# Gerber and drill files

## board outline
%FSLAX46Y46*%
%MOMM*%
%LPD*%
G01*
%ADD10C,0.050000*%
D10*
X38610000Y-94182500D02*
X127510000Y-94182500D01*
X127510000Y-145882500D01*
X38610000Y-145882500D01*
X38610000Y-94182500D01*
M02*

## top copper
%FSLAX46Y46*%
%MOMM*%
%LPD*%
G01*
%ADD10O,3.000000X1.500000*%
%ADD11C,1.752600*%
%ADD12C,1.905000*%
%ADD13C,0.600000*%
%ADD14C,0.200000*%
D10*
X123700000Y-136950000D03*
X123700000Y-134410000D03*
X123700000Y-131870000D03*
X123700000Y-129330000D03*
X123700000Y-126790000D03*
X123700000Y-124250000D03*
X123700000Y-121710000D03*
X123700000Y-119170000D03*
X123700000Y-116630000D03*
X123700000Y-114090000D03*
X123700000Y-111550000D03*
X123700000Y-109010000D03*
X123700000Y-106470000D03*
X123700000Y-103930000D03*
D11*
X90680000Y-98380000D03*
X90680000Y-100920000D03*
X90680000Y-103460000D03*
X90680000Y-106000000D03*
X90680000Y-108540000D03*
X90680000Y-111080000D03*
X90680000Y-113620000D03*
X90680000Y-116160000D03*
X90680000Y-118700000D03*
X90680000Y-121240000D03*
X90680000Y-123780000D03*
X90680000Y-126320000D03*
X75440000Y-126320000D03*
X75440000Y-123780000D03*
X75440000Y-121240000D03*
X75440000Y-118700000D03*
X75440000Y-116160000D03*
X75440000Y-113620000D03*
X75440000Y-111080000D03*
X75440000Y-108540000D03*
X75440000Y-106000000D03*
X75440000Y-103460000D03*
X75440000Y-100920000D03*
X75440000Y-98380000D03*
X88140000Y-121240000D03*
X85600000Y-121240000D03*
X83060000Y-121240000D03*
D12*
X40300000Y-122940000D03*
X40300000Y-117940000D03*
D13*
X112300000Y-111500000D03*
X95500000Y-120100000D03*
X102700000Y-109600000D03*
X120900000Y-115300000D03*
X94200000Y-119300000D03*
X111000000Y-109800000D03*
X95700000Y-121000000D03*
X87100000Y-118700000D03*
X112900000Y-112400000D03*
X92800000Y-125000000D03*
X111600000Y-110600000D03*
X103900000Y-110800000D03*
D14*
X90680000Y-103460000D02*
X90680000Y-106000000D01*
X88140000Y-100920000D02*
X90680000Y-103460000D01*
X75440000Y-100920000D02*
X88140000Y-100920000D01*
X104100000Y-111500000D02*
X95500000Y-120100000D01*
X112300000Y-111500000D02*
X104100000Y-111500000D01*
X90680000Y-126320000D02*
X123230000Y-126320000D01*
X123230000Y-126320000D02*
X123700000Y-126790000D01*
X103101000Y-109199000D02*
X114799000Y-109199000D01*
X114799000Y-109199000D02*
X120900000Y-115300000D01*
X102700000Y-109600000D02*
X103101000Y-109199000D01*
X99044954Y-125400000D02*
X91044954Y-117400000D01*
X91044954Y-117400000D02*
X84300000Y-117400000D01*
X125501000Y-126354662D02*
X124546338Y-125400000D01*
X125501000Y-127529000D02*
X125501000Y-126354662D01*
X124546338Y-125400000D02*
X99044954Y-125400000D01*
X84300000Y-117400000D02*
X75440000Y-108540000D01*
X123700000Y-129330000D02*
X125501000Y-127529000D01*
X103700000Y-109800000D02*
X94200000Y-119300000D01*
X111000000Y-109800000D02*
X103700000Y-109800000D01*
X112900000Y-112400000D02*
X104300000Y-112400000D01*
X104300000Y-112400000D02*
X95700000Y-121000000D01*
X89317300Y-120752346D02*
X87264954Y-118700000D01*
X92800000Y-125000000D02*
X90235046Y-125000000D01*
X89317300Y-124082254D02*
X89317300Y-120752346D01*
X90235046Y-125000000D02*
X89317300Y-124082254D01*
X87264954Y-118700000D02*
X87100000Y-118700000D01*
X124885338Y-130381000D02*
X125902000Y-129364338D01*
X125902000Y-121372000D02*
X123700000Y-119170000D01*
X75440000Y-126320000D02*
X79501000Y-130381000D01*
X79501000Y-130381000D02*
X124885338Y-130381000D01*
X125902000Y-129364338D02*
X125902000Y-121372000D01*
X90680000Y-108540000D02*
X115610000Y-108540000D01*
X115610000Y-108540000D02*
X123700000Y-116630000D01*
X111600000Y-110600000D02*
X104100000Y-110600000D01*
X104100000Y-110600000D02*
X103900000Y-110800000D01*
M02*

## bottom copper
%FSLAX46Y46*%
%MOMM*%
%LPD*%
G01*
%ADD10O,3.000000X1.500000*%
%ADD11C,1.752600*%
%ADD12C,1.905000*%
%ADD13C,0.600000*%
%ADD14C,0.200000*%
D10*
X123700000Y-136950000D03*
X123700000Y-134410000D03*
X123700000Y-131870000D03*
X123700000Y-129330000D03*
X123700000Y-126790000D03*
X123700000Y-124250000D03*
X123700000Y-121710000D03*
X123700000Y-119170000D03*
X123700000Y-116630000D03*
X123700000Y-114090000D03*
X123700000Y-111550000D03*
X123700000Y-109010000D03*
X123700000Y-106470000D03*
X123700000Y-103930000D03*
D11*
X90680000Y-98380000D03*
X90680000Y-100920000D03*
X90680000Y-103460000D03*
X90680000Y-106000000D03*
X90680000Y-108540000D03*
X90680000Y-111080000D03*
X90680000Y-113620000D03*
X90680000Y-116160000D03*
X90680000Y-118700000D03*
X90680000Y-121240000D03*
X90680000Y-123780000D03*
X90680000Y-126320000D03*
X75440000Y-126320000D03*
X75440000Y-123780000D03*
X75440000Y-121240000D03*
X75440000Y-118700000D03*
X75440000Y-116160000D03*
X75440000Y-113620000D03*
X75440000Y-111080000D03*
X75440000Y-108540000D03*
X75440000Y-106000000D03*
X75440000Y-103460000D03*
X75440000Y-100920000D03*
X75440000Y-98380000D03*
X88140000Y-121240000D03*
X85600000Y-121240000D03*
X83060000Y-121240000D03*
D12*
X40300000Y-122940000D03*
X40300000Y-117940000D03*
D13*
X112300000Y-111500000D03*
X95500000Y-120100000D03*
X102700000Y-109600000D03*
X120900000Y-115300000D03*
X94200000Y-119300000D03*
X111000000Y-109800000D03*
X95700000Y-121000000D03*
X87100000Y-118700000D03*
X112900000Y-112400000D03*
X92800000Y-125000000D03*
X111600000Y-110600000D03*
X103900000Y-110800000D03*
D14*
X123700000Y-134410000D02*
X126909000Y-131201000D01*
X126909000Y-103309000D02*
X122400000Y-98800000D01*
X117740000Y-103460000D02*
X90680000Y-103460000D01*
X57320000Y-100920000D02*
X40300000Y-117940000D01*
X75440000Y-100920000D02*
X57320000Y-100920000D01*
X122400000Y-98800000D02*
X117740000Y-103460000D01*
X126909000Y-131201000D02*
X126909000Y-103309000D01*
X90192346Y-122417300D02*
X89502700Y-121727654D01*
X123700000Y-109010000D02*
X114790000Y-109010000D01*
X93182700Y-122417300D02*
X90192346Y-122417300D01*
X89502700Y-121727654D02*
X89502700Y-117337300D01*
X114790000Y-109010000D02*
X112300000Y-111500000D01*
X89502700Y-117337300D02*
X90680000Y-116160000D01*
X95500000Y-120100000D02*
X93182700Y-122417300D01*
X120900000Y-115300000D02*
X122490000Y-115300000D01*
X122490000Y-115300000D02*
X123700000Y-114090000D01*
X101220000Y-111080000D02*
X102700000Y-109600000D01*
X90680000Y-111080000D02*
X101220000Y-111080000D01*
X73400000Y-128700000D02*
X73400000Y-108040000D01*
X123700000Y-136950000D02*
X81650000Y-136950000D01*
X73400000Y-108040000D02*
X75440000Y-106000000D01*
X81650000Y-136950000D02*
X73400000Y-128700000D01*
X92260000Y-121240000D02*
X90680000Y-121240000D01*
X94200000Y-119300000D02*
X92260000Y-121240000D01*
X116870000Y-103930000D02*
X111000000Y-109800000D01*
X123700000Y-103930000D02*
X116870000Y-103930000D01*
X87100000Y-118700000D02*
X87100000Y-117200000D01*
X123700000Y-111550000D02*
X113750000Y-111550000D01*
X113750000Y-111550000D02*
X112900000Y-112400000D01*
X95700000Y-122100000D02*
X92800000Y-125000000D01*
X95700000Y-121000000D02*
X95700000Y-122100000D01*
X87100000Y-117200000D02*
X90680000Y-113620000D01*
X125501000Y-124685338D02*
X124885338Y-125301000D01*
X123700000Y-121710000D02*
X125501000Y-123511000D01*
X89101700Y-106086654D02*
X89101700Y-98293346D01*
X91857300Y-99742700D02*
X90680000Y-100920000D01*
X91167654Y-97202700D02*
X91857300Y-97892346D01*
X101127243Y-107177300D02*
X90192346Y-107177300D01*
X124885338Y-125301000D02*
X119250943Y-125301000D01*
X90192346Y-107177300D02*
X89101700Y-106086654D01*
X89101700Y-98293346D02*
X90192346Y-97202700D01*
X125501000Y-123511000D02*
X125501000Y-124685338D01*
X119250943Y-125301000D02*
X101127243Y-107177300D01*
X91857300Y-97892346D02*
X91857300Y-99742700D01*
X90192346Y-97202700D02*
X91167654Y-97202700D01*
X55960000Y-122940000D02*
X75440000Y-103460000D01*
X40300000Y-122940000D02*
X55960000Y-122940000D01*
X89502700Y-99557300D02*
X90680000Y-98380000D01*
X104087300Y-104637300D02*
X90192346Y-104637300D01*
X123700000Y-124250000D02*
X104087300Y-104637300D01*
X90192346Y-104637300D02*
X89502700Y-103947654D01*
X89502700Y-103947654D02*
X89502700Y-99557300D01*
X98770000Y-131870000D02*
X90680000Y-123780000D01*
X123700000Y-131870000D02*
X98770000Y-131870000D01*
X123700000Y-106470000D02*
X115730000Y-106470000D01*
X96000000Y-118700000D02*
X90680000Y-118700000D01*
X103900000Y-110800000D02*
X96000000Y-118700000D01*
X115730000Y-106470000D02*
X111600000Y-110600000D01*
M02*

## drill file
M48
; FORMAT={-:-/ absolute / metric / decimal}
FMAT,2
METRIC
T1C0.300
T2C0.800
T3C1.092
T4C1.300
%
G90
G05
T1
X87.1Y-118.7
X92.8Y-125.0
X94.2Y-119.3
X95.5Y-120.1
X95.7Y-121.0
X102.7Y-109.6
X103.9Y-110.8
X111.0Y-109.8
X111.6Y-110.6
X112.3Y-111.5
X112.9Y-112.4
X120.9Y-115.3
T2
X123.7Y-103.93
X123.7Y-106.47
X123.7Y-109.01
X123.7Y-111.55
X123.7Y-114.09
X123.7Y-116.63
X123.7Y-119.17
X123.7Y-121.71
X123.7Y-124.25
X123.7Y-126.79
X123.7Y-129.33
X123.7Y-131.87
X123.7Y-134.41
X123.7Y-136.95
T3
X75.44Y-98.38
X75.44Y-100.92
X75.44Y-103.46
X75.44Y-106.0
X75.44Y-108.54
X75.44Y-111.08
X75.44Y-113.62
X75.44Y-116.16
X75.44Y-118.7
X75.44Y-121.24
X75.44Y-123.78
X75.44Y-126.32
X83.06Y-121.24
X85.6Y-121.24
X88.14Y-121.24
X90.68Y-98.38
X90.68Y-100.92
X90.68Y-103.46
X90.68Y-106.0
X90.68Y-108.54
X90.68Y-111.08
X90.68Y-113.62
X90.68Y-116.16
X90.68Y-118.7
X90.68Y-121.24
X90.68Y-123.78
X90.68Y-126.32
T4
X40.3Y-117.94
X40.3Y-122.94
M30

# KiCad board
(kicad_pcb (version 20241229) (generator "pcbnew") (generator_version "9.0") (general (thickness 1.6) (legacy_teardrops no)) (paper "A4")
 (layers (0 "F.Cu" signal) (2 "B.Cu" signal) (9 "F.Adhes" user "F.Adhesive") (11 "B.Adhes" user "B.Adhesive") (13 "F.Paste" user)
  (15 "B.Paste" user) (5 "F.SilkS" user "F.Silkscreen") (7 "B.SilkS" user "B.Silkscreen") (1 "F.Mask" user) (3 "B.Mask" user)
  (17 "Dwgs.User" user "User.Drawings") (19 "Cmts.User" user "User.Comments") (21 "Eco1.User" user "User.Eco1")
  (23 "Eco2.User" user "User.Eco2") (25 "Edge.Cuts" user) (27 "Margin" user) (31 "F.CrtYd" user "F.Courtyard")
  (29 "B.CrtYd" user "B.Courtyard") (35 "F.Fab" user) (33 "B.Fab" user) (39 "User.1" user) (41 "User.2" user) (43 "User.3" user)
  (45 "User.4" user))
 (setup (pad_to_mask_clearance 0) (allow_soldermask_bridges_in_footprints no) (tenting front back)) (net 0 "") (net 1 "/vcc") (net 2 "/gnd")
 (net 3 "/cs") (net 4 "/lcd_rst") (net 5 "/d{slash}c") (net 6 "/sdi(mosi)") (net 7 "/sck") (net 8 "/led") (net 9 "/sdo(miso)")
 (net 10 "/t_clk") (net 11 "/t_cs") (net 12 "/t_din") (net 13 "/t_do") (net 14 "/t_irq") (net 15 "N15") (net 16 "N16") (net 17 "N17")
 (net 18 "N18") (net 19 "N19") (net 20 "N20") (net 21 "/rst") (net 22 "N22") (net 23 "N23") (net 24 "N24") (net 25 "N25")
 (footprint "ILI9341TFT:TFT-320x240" (layer "F.Cu") (at 123.7 120.44 90)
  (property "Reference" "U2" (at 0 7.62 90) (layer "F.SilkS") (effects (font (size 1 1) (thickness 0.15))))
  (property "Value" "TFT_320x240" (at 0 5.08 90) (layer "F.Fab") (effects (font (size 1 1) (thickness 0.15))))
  (pad "1" thru_hole oval (at -16.51 0 90) (size 1.5 3) (drill 0.8) (layers "*.Cu" "*.Mask") (remove_unused_layers no) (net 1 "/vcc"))
  (pad "2" thru_hole oval (at -13.97 0 90) (size 1.5 3) (drill 0.8) (layers "*.Cu" "*.Mask") (remove_unused_layers no) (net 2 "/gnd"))
  (pad "3" thru_hole oval (at -11.43 0 90) (size 1.5 3) (drill 0.8) (layers "*.Cu" "*.Mask") (remove_unused_layers no) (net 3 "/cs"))
  (pad "4" thru_hole oval (at -8.89 0 90) (size 1.5 3) (drill 0.8) (layers "*.Cu" "*.Mask") (remove_unused_layers no) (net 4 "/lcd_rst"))
  (pad "5" thru_hole oval (at -6.35 0 90) (size 1.5 3) (drill 0.8) (layers "*.Cu" "*.Mask") (remove_unused_layers no) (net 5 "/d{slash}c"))
  (pad "6" thru_hole oval (at -3.81 0 90) (size 1.5 3) (drill 0.8) (layers "*.Cu" "*.Mask") (remove_unused_layers no) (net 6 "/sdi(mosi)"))
  (pad "7" thru_hole oval (at -1.27 0 90) (size 1.5 3) (drill 0.8) (layers "*.Cu" "*.Mask") (remove_unused_layers no) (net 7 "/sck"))
  (pad "8" thru_hole oval (at 1.27 0 90) (size 1.5 3) (drill 0.8) (layers "*.Cu" "*.Mask") (remove_unused_layers no) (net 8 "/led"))
  (pad "9" thru_hole oval (at 3.81 0 90) (size 1.5 3) (drill 0.8) (layers "*.Cu" "*.Mask") (remove_unused_layers no) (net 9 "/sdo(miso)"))
  (pad "10" thru_hole oval (at 6.35 0 90) (size 1.5 3) (drill 0.8) (layers "*.Cu" "*.Mask") (remove_unused_layers no) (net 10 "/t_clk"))
  (pad "11" thru_hole oval (at 8.89 0 90) (size 1.5 3) (drill 0.8) (layers "*.Cu" "*.Mask") (remove_unused_layers no) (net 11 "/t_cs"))
  (pad "12" thru_hole oval (at 11.43 0 90) (size 1.5 3) (drill 0.8) (layers "*.Cu" "*.Mask") (remove_unused_layers no) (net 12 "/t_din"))
  (pad "13" thru_hole oval (at 13.97 0 90) (size 1.5 3) (drill 0.8) (layers "*.Cu" "*.Mask") (remove_unused_layers no) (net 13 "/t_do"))
  (pad "14" thru_hole oval (at 16.51 0 90) (size 1.5 3) (drill 0.8) (layers "*.Cu" "*.Mask") (remove_unused_layers no) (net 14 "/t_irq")))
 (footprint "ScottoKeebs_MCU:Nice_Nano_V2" (layer "B.Cu") (at 83.06 112.07 180)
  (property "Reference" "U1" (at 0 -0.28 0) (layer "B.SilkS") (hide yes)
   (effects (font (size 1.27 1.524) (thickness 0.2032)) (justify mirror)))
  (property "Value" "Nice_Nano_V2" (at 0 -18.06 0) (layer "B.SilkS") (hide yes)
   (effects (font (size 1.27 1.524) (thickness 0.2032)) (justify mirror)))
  (pad "1" thru_hole circle (at -7.62 13.69 270) (size 1.7526 1.7526) (drill 1.0922) (layers "*.Cu" "*.Mask") (remove_unused_layers no)
   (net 6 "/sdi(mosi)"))
  (pad "2" thru_hole circle (at -7.62 11.15 270) (size 1.7526 1.7526) (drill 1.0922) (layers "*.Cu" "*.Mask") (remove_unused_layers no)
   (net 7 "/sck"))
  (pad "3" thru_hole circle (at -7.62 8.61 270) (size 1.7526 1.7526) (drill 1.0922) (layers "*.Cu" "*.Mask") (remove_unused_layers no)
   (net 2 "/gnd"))
  (pad "4" thru_hole circle (at -7.62 6.07 270) (size 1.7526 1.7526) (drill 1.0922) (layers "*.Cu" "*.Mask") (remove_unused_layers no)
   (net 2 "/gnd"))
  (pad "5" thru_hole circle (at -7.62 3.53 270) (size 1.7526 1.7526) (drill 1.0922) (layers "*.Cu" "*.Mask") (remove_unused_layers no)
   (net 9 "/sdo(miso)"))
  (pad "6" thru_hole circle (at -7.62 0.99 270) (size 1.7526 1.7526) (drill 1.0922) (layers "*.Cu" "*.Mask") (remove_unused_layers no)
   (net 10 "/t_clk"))
  (pad "7" thru_hole circle (at -7.62 -1.55 270) (size 1.7526 1.7526) (drill 1.0922) (layers "*.Cu" "*.Mask") (remove_unused_layers no)
   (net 11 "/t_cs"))
  (pad "8" thru_hole circle (at -7.62 -4.09 270) (size 1.7526 1.7526) (drill 1.0922) (layers "*.Cu" "*.Mask") (remove_unused_layers no)
   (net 12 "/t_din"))
  (pad "9" thru_hole circle (at -7.62 -6.63 270) (size 1.7526 1.7526) (drill 1.0922) (layers "*.Cu" "*.Mask") (remove_unused_layers no)
   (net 13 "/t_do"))
  (pad "10" thru_hole circle (at -7.62 -9.17 270) (size 1.7526 1.7526) (drill 1.0922) (layers "*.Cu" "*.Mask") (remove_unused_layers no)
   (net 14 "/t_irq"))
  (pad "11" thru_hole circle (at -7.62 -11.71 270) (size 1.7526 1.7526) (drill 1.0922) (layers "*.Cu" "*.Mask") (remove_unused_layers no)
   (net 3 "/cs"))
  (pad "12" thru_hole circle (at -7.62 -14.25 270) (size 1.7526 1.7526) (drill 1.0922) (layers "*.Cu" "*.Mask") (remove_unused_layers no)
   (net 5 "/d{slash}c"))
  (pad "13" thru_hole circle (at 7.62 -14.25 270) (size 1.7526 1.7526) (drill 1.0922) (layers "*.Cu" "*.Mask") (remove_unused_layers no)
   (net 8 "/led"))
  (pad "14" thru_hole circle (at 7.62 -11.71 270) (size 1.7526 1.7526) (drill 1.0922) (layers "*.Cu" "*.Mask") (remove_unused_layers no)
   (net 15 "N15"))
  (pad "15" thru_hole circle (at 7.62 -9.17 270) (size 1.7526 1.7526) (drill 1.0922) (layers "*.Cu" "*.Mask") (remove_unused_layers no)
   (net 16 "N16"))
  (pad "16" thru_hole circle (at 7.62 -6.63 270) (size 1.7526 1.7526) (drill 1.0922) (layers "*.Cu" "*.Mask") (remove_unused_layers no)
   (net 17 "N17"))
  (pad "17" thru_hole circle (at 7.62 -4.09 270) (size 1.7526 1.7526) (drill 1.0922) (layers "*.Cu" "*.Mask") (remove_unused_layers no)
   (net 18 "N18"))
  (pad "18" thru_hole circle (at 7.62 -1.55 270) (size 1.7526 1.7526) (drill 1.0922) (layers "*.Cu" "*.Mask") (remove_unused_layers no)
   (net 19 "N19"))
  (pad "19" thru_hole circle (at 7.62 0.99 270) (size 1.7526 1.7526) (drill 1.0922) (layers "*.Cu" "*.Mask") (remove_unused_layers no)
   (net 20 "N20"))
  (pad "20" thru_hole circle (at 7.62 3.53 270) (size 1.7526 1.7526) (drill 1.0922) (layers "*.Cu" "*.Mask") (remove_unused_layers no)
   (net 4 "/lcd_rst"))
  (pad "21" thru_hole circle (at 7.62 6.07 270) (size 1.7526 1.7526) (drill 1.0922) (layers "*.Cu" "*.Mask") (remove_unused_layers no)
   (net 1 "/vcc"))
  (pad "22" thru_hole circle (at 7.62 8.61 270) (size 1.7526 1.7526) (drill 1.0922) (layers "*.Cu" "*.Mask") (remove_unused_layers no)
   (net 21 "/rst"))
  (pad "23" thru_hole circle (at 7.62 11.15 270) (size 1.7526 1.7526) (drill 1.0922) (layers "*.Cu" "*.Mask") (remove_unused_layers no)
   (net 2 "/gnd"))
  (pad "24" thru_hole circle (at 7.62 13.69 270) (size 1.7526 1.7526) (drill 1.0922) (layers "*.Cu" "*.Mask") (remove_unused_layers no)
   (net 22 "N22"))
  (pad "25" thru_hole circle (at -5.08 -9.17 180) (size 1.7526 1.7526) (drill 1.0922) (layers "*.Cu" "*.Mask") (remove_unused_layers no)
   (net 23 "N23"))
  (pad "26" thru_hole circle (at -2.54 -9.17 180) (size 1.7526 1.7526) (drill 1.0922) (layers "*.Cu" "*.Mask") (remove_unused_layers no)
   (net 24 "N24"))
  (pad "27" thru_hole circle (at 0 -9.17 180) (size 1.7526 1.7526) (drill 1.0922) (layers "*.Cu" "*.Mask") (remove_unused_layers no)
   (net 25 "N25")))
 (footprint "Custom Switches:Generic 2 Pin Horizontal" (layer "B.Cu") (at 40.3 120.44 90)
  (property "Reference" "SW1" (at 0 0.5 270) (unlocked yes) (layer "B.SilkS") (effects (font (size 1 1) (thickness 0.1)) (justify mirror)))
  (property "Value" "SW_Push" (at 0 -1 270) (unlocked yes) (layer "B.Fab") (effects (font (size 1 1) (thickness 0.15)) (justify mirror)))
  (pad "1" thru_hole circle (at -2.5 0 90) (size 1.905 1.905) (drill 1.3) (layers "*.Cu" "*.Mask") (remove_unused_layers no) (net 21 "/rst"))
  (pad "2" thru_hole circle (at 2.5 0 90) (size 1.905 1.905) (drill 1.3) (layers "*.Cu" "*.Mask") (remove_unused_layers no) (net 2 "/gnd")))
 (gr_rect (start 38.61 94.1825) (end 127.51 145.8825) (stroke (width 0.05) (type default)) (fill no) (layer "Edge.Cuts"))
 (segment (start 90.68 103.46) (end 90.68 106) (width 0.2) (layer "F.Cu") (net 2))
 (segment (start 88.14 100.92) (end 90.68 103.46) (width 0.2) (layer "F.Cu") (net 2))
 (segment (start 75.44 100.92) (end 88.14 100.92) (width 0.2) (layer "F.Cu") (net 2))
 (segment (start 123.7 134.41) (end 126.909 131.201) (width 0.2) (layer "B.Cu") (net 2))
 (segment (start 126.909 103.309) (end 122.4 98.8) (width 0.2) (layer "B.Cu") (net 2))
 (segment (start 117.74 103.46) (end 90.68 103.46) (width 0.2) (layer "B.Cu") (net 2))
 (segment (start 57.32 100.92) (end 40.3 117.94) (width 0.2) (layer "B.Cu") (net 2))
 (segment (start 75.44 100.92) (end 57.32 100.92) (width 0.2) (layer "B.Cu") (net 2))
 (segment (start 122.4 98.8) (end 117.74 103.46) (width 0.2) (layer "B.Cu") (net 2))
 (segment (start 126.909 131.201) (end 126.909 103.309) (width 0.2) (layer "B.Cu") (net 2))
 (segment (start 104.1 111.5) (end 95.5 120.1) (width 0.2) (layer "F.Cu") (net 12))
 (segment (start 112.3 111.5) (end 104.1 111.5) (width 0.2) (layer "F.Cu") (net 12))
 (via (at 112.3 111.5) (size 0.6) (drill 0.3) (layers "F.Cu" "B.Cu") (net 12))
 (via (at 95.5 120.1) (size 0.6) (drill 0.3) (layers "F.Cu" "B.Cu") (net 12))
 (segment (start 90.192346 122.4173) (end 89.5027 121.727654) (width 0.2) (layer "B.Cu") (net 12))
 (segment (start 123.7 109.01) (end 114.79 109.01) (width 0.2) (layer "B.Cu") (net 12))
 (segment (start 93.1827 122.4173) (end 90.192346 122.4173) (width 0.2) (layer "B.Cu") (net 12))
 (segment (start 89.5027 121.727654) (end 89.5027 117.3373) (width 0.2) (layer "B.Cu") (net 12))
 (segment (start 114.79 109.01) (end 112.3 111.5) (width 0.2) (layer "B.Cu") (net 12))
 (segment (start 89.5027 117.3373) (end 90.68 116.16) (width 0.2) (layer "B.Cu") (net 12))
 (segment (start 95.5 120.1) (end 93.1827 122.4173) (width 0.2) (layer "B.Cu") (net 12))
 (segment (start 90.68 126.32) (end 123.23 126.32) (width 0.2) (layer "F.Cu") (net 5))
 (segment (start 123.23 126.32) (end 123.7 126.79) (width 0.2) (layer "F.Cu") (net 5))
 (segment (start 103.101 109.199) (end 114.799 109.199) (width 0.2) (layer "F.Cu") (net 10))
 (segment (start 114.799 109.199) (end 120.9 115.3) (width 0.2) (layer "F.Cu") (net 10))
 (segment (start 102.7 109.6) (end 103.101 109.199) (width 0.2) (layer "F.Cu") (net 10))
 (via (at 102.7 109.6) (size 0.6) (drill 0.3) (layers "F.Cu" "B.Cu") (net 10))
 (via (at 120.9 115.3) (size 0.6) (drill 0.3) (layers "F.Cu" "B.Cu") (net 10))
 (segment (start 120.9 115.3) (end 122.49 115.3) (width 0.2) (layer "B.Cu") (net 10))
 (segment (start 122.49 115.3) (end 123.7 114.09) (width 0.2) (layer "B.Cu") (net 10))
 (segment (start 101.22 111.08) (end 102.7 109.6) (width 0.2) (layer "B.Cu") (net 10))
 (segment (start 90.68 111.08) (end 101.22 111.08) (width 0.2) (layer "B.Cu") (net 10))
 (segment (start 73.4 128.7) (end 73.4 108.04) (width 0.2) (layer "B.Cu") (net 1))
 (segment (start 123.7 136.95) (end 81.65 136.95) (width 0.2) (layer "B.Cu") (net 1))
 (segment (start 73.4 108.04) (end 75.44 106) (width 0.2) (layer "B.Cu") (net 1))
 (segment (start 81.65 136.95) (end 73.4 128.7) (width 0.2) (layer "B.Cu") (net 1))
 (segment (start 99.044954 125.4) (end 91.044954 117.4) (width 0.2) (layer "F.Cu") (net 4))
 (segment (start 91.044954 117.4) (end 84.3 117.4) (width 0.2) (layer "F.Cu") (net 4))
 (segment (start 125.501 126.354662) (end 124.546338 125.4) (width 0.2) (layer "F.Cu") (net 4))
 (segment (start 125.501 127.529) (end 125.501 126.354662) (width 0.2) (layer "F.Cu") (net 4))
 (segment (start 124.546338 125.4) (end 99.044954 125.4) (width 0.2) (layer "F.Cu") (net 4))
 (segment (start 84.3 117.4) (end 75.44 108.54) (width 0.2) (layer "F.Cu") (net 4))
 (segment (start 123.7 129.33) (end 125.501 127.529) (width 0.2) (layer "F.Cu") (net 4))
 (segment (start 103.7 109.8) (end 94.2 119.3) (width 0.2) (layer "F.Cu") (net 14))
 (segment (start 111 109.8) (end 103.7 109.8) (width 0.2) (layer "F.Cu") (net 14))
 (via (at 94.2 119.3) (size 0.6) (drill 0.3) (layers "F.Cu" "B.Cu") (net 14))
 (via (at 111 109.8) (size 0.6) (drill 0.3) (layers "F.Cu" "B.Cu") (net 14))
 (segment (start 92.26 121.24) (end 90.68 121.24) (width 0.2) (layer "B.Cu") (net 14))
 (segment (start 94.2 119.3) (end 92.26 121.24) (width 0.2) (layer "B.Cu") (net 14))
 (segment (start 116.87 103.93) (end 111 109.8) (width 0.2) (layer "B.Cu") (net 14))
 (segment (start 123.7 103.93) (end 116.87 103.93) (width 0.2) (layer "B.Cu") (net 14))
 (segment (start 112.9 112.4) (end 104.3 112.4) (width 0.2) (layer "F.Cu") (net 11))
 (segment (start 104.3 112.4) (end 95.7 121) (width 0.2) (layer "F.Cu") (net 11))
 (segment (start 89.3173 120.752346) (end 87.264954 118.7) (width 0.2) (layer "F.Cu") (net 11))
 (segment (start 92.8 125) (end 90.235046 125) (width 0.2) (layer "F.Cu") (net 11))
 (segment (start 89.3173 124.082254) (end 89.3173 120.752346) (width 0.2) (layer "F.Cu") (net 11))
 (segment (start 90.235046 125) (end 89.3173 124.082254) (width 0.2) (layer "F.Cu") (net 11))
 (segment (start 87.264954 118.7) (end 87.1 118.7) (width 0.2) (layer "F.Cu") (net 11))
 (via (at 95.7 121) (size 0.6) (drill 0.3) (layers "F.Cu" "B.Cu") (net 11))
 (via (at 87.1 118.7) (size 0.6) (drill 0.3) (layers "F.Cu" "B.Cu") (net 11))
 (via (at 112.9 112.4) (size 0.6) (drill 0.3) (layers "F.Cu" "B.Cu") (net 11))
 (via (at 92.8 125) (size 0.6) (drill 0.3) (layers "F.Cu" "B.Cu") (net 11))
 (segment (start 87.1 118.7) (end 87.1 117.2) (width 0.2) (layer "B.Cu") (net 11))
 (segment (start 123.7 111.55) (end 113.75 111.55) (width 0.2) (layer "B.Cu") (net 11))
 (segment (start 113.75 111.55) (end 112.9 112.4) (width 0.2) (layer "B.Cu") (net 11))
 (segment (start 95.7 122.1) (end 92.8 125) (width 0.2) (layer "B.Cu") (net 11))
 (segment (start 95.7 121) (end 95.7 122.1) (width 0.2) (layer "B.Cu") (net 11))
 (segment (start 87.1 117.2) (end 90.68 113.62) (width 0.2) (layer "B.Cu") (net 11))
 (segment (start 125.501 124.685338) (end 124.885338 125.301) (width 0.2) (layer "B.Cu") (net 7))
 (segment (start 123.7 121.71) (end 125.501 123.511) (width 0.2) (layer "B.Cu") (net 7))
 (segment (start 89.1017 106.086654) (end 89.1017 98.293346) (width 0.2) (layer "B.Cu") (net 7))
 (segment (start 91.8573 99.7427) (end 90.68 100.92) (width 0.2) (layer "B.Cu") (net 7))
 (segment (start 91.167654 97.2027) (end 91.8573 97.892346) (width 0.2) (layer "B.Cu") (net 7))
 (segment (start 101.127243 107.1773) (end 90.192346 107.1773) (width 0.2) (layer "B.Cu") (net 7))
 (segment (start 124.885338 125.301) (end 119.250943 125.301) (width 0.2) (layer "B.Cu") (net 7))
 (segment (start 90.192346 107.1773) (end 89.1017 106.086654) (width 0.2) (layer "B.Cu") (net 7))
 (segment (start 89.1017 98.293346) (end 90.192346 97.2027) (width 0.2) (layer "B.Cu") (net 7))
 (segment (start 125.501 123.511) (end 125.501 124.685338) (width 0.2) (layer "B.Cu") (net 7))
 (segment (start 119.250943 125.301) (end 101.127243 107.1773) (width 0.2) (layer "B.Cu") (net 7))
 (segment (start 91.8573 97.892346) (end 91.8573 99.7427) (width 0.2) (layer "B.Cu") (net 7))
 (segment (start 90.192346 97.2027) (end 91.167654 97.2027) (width 0.2) (layer "B.Cu") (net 7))
 (segment (start 55.96 122.94) (end 75.44 103.46) (width 0.2) (layer "B.Cu") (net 21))
 (segment (start 40.3 122.94) (end 55.96 122.94) (width 0.2) (layer "B.Cu") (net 21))
 (segment (start 89.5027 99.5573) (end 90.68 98.38) (width 0.2) (layer "B.Cu") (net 6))
 (segment (start 104.0873 104.6373) (end 90.192346 104.6373) (width 0.2) (layer "B.Cu") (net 6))
 (segment (start 123.7 124.25) (end 104.0873 104.6373) (width 0.2) (layer "B.Cu") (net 6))
 (segment (start 90.192346 104.6373) (end 89.5027 103.947654) (width 0.2) (layer "B.Cu") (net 6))
 (segment (start 89.5027 103.947654) (end 89.5027 99.5573) (width 0.2) (layer "B.Cu") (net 6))
 (segment (start 124.885338 130.381) (end 125.902 129.364338) (width 0.2) (layer "F.Cu") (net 8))
 (segment (start 125.902 121.372) (end 123.7 119.17) (width 0.2) (layer "F.Cu") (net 8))
 (segment (start 75.44 126.32) (end 79.501 130.381) (width 0.2) (layer "F.Cu") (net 8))
 (segment (start 79.501 130.381) (end 124.885338 130.381) (width 0.2) (layer "F.Cu") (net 8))
 (segment (start 125.902 129.364338) (end 125.902 121.372) (width 0.2) (layer "F.Cu") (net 8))
 (segment (start 90.68 108.54) (end 115.61 108.54) (width 0.2) (layer "F.Cu") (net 9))
 (segment (start 115.61 108.54) (end 123.7 116.63) (width 0.2) (layer "F.Cu") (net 9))
 (segment (start 98.77 131.87) (end 90.68 123.78) (width 0.2) (layer "B.Cu") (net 3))
 (segment (start 123.7 131.87) (end 98.77 131.87) (width 0.2) (layer "B.Cu") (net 3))
 (segment (start 111.6 110.6) (end 104.1 110.6) (width 0.2) (layer "F.Cu") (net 13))
 (segment (start 104.1 110.6) (end 103.9 110.8) (width 0.2) (layer "F.Cu") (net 13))
 (via (at 111.6 110.6) (size 0.6) (drill 0.3) (layers "F.Cu" "B.Cu") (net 13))
 (via (at 103.9 110.8) (size 0.6) (drill 0.3) (layers "F.Cu" "B.Cu") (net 13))
 (segment (start 123.7 106.47) (end 115.73 106.47) (width 0.2) (layer "B.Cu") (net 13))
 (segment (start 96 118.7) (end 90.68 118.7) (width 0.2) (layer "B.Cu") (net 13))
 (segment (start 103.9 110.8) (end 96 118.7) (width 0.2) (layer "B.Cu") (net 13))
 (segment (start 115.73 106.47) (end 111.6 110.6) (width 0.2) (layer "B.Cu") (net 13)))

